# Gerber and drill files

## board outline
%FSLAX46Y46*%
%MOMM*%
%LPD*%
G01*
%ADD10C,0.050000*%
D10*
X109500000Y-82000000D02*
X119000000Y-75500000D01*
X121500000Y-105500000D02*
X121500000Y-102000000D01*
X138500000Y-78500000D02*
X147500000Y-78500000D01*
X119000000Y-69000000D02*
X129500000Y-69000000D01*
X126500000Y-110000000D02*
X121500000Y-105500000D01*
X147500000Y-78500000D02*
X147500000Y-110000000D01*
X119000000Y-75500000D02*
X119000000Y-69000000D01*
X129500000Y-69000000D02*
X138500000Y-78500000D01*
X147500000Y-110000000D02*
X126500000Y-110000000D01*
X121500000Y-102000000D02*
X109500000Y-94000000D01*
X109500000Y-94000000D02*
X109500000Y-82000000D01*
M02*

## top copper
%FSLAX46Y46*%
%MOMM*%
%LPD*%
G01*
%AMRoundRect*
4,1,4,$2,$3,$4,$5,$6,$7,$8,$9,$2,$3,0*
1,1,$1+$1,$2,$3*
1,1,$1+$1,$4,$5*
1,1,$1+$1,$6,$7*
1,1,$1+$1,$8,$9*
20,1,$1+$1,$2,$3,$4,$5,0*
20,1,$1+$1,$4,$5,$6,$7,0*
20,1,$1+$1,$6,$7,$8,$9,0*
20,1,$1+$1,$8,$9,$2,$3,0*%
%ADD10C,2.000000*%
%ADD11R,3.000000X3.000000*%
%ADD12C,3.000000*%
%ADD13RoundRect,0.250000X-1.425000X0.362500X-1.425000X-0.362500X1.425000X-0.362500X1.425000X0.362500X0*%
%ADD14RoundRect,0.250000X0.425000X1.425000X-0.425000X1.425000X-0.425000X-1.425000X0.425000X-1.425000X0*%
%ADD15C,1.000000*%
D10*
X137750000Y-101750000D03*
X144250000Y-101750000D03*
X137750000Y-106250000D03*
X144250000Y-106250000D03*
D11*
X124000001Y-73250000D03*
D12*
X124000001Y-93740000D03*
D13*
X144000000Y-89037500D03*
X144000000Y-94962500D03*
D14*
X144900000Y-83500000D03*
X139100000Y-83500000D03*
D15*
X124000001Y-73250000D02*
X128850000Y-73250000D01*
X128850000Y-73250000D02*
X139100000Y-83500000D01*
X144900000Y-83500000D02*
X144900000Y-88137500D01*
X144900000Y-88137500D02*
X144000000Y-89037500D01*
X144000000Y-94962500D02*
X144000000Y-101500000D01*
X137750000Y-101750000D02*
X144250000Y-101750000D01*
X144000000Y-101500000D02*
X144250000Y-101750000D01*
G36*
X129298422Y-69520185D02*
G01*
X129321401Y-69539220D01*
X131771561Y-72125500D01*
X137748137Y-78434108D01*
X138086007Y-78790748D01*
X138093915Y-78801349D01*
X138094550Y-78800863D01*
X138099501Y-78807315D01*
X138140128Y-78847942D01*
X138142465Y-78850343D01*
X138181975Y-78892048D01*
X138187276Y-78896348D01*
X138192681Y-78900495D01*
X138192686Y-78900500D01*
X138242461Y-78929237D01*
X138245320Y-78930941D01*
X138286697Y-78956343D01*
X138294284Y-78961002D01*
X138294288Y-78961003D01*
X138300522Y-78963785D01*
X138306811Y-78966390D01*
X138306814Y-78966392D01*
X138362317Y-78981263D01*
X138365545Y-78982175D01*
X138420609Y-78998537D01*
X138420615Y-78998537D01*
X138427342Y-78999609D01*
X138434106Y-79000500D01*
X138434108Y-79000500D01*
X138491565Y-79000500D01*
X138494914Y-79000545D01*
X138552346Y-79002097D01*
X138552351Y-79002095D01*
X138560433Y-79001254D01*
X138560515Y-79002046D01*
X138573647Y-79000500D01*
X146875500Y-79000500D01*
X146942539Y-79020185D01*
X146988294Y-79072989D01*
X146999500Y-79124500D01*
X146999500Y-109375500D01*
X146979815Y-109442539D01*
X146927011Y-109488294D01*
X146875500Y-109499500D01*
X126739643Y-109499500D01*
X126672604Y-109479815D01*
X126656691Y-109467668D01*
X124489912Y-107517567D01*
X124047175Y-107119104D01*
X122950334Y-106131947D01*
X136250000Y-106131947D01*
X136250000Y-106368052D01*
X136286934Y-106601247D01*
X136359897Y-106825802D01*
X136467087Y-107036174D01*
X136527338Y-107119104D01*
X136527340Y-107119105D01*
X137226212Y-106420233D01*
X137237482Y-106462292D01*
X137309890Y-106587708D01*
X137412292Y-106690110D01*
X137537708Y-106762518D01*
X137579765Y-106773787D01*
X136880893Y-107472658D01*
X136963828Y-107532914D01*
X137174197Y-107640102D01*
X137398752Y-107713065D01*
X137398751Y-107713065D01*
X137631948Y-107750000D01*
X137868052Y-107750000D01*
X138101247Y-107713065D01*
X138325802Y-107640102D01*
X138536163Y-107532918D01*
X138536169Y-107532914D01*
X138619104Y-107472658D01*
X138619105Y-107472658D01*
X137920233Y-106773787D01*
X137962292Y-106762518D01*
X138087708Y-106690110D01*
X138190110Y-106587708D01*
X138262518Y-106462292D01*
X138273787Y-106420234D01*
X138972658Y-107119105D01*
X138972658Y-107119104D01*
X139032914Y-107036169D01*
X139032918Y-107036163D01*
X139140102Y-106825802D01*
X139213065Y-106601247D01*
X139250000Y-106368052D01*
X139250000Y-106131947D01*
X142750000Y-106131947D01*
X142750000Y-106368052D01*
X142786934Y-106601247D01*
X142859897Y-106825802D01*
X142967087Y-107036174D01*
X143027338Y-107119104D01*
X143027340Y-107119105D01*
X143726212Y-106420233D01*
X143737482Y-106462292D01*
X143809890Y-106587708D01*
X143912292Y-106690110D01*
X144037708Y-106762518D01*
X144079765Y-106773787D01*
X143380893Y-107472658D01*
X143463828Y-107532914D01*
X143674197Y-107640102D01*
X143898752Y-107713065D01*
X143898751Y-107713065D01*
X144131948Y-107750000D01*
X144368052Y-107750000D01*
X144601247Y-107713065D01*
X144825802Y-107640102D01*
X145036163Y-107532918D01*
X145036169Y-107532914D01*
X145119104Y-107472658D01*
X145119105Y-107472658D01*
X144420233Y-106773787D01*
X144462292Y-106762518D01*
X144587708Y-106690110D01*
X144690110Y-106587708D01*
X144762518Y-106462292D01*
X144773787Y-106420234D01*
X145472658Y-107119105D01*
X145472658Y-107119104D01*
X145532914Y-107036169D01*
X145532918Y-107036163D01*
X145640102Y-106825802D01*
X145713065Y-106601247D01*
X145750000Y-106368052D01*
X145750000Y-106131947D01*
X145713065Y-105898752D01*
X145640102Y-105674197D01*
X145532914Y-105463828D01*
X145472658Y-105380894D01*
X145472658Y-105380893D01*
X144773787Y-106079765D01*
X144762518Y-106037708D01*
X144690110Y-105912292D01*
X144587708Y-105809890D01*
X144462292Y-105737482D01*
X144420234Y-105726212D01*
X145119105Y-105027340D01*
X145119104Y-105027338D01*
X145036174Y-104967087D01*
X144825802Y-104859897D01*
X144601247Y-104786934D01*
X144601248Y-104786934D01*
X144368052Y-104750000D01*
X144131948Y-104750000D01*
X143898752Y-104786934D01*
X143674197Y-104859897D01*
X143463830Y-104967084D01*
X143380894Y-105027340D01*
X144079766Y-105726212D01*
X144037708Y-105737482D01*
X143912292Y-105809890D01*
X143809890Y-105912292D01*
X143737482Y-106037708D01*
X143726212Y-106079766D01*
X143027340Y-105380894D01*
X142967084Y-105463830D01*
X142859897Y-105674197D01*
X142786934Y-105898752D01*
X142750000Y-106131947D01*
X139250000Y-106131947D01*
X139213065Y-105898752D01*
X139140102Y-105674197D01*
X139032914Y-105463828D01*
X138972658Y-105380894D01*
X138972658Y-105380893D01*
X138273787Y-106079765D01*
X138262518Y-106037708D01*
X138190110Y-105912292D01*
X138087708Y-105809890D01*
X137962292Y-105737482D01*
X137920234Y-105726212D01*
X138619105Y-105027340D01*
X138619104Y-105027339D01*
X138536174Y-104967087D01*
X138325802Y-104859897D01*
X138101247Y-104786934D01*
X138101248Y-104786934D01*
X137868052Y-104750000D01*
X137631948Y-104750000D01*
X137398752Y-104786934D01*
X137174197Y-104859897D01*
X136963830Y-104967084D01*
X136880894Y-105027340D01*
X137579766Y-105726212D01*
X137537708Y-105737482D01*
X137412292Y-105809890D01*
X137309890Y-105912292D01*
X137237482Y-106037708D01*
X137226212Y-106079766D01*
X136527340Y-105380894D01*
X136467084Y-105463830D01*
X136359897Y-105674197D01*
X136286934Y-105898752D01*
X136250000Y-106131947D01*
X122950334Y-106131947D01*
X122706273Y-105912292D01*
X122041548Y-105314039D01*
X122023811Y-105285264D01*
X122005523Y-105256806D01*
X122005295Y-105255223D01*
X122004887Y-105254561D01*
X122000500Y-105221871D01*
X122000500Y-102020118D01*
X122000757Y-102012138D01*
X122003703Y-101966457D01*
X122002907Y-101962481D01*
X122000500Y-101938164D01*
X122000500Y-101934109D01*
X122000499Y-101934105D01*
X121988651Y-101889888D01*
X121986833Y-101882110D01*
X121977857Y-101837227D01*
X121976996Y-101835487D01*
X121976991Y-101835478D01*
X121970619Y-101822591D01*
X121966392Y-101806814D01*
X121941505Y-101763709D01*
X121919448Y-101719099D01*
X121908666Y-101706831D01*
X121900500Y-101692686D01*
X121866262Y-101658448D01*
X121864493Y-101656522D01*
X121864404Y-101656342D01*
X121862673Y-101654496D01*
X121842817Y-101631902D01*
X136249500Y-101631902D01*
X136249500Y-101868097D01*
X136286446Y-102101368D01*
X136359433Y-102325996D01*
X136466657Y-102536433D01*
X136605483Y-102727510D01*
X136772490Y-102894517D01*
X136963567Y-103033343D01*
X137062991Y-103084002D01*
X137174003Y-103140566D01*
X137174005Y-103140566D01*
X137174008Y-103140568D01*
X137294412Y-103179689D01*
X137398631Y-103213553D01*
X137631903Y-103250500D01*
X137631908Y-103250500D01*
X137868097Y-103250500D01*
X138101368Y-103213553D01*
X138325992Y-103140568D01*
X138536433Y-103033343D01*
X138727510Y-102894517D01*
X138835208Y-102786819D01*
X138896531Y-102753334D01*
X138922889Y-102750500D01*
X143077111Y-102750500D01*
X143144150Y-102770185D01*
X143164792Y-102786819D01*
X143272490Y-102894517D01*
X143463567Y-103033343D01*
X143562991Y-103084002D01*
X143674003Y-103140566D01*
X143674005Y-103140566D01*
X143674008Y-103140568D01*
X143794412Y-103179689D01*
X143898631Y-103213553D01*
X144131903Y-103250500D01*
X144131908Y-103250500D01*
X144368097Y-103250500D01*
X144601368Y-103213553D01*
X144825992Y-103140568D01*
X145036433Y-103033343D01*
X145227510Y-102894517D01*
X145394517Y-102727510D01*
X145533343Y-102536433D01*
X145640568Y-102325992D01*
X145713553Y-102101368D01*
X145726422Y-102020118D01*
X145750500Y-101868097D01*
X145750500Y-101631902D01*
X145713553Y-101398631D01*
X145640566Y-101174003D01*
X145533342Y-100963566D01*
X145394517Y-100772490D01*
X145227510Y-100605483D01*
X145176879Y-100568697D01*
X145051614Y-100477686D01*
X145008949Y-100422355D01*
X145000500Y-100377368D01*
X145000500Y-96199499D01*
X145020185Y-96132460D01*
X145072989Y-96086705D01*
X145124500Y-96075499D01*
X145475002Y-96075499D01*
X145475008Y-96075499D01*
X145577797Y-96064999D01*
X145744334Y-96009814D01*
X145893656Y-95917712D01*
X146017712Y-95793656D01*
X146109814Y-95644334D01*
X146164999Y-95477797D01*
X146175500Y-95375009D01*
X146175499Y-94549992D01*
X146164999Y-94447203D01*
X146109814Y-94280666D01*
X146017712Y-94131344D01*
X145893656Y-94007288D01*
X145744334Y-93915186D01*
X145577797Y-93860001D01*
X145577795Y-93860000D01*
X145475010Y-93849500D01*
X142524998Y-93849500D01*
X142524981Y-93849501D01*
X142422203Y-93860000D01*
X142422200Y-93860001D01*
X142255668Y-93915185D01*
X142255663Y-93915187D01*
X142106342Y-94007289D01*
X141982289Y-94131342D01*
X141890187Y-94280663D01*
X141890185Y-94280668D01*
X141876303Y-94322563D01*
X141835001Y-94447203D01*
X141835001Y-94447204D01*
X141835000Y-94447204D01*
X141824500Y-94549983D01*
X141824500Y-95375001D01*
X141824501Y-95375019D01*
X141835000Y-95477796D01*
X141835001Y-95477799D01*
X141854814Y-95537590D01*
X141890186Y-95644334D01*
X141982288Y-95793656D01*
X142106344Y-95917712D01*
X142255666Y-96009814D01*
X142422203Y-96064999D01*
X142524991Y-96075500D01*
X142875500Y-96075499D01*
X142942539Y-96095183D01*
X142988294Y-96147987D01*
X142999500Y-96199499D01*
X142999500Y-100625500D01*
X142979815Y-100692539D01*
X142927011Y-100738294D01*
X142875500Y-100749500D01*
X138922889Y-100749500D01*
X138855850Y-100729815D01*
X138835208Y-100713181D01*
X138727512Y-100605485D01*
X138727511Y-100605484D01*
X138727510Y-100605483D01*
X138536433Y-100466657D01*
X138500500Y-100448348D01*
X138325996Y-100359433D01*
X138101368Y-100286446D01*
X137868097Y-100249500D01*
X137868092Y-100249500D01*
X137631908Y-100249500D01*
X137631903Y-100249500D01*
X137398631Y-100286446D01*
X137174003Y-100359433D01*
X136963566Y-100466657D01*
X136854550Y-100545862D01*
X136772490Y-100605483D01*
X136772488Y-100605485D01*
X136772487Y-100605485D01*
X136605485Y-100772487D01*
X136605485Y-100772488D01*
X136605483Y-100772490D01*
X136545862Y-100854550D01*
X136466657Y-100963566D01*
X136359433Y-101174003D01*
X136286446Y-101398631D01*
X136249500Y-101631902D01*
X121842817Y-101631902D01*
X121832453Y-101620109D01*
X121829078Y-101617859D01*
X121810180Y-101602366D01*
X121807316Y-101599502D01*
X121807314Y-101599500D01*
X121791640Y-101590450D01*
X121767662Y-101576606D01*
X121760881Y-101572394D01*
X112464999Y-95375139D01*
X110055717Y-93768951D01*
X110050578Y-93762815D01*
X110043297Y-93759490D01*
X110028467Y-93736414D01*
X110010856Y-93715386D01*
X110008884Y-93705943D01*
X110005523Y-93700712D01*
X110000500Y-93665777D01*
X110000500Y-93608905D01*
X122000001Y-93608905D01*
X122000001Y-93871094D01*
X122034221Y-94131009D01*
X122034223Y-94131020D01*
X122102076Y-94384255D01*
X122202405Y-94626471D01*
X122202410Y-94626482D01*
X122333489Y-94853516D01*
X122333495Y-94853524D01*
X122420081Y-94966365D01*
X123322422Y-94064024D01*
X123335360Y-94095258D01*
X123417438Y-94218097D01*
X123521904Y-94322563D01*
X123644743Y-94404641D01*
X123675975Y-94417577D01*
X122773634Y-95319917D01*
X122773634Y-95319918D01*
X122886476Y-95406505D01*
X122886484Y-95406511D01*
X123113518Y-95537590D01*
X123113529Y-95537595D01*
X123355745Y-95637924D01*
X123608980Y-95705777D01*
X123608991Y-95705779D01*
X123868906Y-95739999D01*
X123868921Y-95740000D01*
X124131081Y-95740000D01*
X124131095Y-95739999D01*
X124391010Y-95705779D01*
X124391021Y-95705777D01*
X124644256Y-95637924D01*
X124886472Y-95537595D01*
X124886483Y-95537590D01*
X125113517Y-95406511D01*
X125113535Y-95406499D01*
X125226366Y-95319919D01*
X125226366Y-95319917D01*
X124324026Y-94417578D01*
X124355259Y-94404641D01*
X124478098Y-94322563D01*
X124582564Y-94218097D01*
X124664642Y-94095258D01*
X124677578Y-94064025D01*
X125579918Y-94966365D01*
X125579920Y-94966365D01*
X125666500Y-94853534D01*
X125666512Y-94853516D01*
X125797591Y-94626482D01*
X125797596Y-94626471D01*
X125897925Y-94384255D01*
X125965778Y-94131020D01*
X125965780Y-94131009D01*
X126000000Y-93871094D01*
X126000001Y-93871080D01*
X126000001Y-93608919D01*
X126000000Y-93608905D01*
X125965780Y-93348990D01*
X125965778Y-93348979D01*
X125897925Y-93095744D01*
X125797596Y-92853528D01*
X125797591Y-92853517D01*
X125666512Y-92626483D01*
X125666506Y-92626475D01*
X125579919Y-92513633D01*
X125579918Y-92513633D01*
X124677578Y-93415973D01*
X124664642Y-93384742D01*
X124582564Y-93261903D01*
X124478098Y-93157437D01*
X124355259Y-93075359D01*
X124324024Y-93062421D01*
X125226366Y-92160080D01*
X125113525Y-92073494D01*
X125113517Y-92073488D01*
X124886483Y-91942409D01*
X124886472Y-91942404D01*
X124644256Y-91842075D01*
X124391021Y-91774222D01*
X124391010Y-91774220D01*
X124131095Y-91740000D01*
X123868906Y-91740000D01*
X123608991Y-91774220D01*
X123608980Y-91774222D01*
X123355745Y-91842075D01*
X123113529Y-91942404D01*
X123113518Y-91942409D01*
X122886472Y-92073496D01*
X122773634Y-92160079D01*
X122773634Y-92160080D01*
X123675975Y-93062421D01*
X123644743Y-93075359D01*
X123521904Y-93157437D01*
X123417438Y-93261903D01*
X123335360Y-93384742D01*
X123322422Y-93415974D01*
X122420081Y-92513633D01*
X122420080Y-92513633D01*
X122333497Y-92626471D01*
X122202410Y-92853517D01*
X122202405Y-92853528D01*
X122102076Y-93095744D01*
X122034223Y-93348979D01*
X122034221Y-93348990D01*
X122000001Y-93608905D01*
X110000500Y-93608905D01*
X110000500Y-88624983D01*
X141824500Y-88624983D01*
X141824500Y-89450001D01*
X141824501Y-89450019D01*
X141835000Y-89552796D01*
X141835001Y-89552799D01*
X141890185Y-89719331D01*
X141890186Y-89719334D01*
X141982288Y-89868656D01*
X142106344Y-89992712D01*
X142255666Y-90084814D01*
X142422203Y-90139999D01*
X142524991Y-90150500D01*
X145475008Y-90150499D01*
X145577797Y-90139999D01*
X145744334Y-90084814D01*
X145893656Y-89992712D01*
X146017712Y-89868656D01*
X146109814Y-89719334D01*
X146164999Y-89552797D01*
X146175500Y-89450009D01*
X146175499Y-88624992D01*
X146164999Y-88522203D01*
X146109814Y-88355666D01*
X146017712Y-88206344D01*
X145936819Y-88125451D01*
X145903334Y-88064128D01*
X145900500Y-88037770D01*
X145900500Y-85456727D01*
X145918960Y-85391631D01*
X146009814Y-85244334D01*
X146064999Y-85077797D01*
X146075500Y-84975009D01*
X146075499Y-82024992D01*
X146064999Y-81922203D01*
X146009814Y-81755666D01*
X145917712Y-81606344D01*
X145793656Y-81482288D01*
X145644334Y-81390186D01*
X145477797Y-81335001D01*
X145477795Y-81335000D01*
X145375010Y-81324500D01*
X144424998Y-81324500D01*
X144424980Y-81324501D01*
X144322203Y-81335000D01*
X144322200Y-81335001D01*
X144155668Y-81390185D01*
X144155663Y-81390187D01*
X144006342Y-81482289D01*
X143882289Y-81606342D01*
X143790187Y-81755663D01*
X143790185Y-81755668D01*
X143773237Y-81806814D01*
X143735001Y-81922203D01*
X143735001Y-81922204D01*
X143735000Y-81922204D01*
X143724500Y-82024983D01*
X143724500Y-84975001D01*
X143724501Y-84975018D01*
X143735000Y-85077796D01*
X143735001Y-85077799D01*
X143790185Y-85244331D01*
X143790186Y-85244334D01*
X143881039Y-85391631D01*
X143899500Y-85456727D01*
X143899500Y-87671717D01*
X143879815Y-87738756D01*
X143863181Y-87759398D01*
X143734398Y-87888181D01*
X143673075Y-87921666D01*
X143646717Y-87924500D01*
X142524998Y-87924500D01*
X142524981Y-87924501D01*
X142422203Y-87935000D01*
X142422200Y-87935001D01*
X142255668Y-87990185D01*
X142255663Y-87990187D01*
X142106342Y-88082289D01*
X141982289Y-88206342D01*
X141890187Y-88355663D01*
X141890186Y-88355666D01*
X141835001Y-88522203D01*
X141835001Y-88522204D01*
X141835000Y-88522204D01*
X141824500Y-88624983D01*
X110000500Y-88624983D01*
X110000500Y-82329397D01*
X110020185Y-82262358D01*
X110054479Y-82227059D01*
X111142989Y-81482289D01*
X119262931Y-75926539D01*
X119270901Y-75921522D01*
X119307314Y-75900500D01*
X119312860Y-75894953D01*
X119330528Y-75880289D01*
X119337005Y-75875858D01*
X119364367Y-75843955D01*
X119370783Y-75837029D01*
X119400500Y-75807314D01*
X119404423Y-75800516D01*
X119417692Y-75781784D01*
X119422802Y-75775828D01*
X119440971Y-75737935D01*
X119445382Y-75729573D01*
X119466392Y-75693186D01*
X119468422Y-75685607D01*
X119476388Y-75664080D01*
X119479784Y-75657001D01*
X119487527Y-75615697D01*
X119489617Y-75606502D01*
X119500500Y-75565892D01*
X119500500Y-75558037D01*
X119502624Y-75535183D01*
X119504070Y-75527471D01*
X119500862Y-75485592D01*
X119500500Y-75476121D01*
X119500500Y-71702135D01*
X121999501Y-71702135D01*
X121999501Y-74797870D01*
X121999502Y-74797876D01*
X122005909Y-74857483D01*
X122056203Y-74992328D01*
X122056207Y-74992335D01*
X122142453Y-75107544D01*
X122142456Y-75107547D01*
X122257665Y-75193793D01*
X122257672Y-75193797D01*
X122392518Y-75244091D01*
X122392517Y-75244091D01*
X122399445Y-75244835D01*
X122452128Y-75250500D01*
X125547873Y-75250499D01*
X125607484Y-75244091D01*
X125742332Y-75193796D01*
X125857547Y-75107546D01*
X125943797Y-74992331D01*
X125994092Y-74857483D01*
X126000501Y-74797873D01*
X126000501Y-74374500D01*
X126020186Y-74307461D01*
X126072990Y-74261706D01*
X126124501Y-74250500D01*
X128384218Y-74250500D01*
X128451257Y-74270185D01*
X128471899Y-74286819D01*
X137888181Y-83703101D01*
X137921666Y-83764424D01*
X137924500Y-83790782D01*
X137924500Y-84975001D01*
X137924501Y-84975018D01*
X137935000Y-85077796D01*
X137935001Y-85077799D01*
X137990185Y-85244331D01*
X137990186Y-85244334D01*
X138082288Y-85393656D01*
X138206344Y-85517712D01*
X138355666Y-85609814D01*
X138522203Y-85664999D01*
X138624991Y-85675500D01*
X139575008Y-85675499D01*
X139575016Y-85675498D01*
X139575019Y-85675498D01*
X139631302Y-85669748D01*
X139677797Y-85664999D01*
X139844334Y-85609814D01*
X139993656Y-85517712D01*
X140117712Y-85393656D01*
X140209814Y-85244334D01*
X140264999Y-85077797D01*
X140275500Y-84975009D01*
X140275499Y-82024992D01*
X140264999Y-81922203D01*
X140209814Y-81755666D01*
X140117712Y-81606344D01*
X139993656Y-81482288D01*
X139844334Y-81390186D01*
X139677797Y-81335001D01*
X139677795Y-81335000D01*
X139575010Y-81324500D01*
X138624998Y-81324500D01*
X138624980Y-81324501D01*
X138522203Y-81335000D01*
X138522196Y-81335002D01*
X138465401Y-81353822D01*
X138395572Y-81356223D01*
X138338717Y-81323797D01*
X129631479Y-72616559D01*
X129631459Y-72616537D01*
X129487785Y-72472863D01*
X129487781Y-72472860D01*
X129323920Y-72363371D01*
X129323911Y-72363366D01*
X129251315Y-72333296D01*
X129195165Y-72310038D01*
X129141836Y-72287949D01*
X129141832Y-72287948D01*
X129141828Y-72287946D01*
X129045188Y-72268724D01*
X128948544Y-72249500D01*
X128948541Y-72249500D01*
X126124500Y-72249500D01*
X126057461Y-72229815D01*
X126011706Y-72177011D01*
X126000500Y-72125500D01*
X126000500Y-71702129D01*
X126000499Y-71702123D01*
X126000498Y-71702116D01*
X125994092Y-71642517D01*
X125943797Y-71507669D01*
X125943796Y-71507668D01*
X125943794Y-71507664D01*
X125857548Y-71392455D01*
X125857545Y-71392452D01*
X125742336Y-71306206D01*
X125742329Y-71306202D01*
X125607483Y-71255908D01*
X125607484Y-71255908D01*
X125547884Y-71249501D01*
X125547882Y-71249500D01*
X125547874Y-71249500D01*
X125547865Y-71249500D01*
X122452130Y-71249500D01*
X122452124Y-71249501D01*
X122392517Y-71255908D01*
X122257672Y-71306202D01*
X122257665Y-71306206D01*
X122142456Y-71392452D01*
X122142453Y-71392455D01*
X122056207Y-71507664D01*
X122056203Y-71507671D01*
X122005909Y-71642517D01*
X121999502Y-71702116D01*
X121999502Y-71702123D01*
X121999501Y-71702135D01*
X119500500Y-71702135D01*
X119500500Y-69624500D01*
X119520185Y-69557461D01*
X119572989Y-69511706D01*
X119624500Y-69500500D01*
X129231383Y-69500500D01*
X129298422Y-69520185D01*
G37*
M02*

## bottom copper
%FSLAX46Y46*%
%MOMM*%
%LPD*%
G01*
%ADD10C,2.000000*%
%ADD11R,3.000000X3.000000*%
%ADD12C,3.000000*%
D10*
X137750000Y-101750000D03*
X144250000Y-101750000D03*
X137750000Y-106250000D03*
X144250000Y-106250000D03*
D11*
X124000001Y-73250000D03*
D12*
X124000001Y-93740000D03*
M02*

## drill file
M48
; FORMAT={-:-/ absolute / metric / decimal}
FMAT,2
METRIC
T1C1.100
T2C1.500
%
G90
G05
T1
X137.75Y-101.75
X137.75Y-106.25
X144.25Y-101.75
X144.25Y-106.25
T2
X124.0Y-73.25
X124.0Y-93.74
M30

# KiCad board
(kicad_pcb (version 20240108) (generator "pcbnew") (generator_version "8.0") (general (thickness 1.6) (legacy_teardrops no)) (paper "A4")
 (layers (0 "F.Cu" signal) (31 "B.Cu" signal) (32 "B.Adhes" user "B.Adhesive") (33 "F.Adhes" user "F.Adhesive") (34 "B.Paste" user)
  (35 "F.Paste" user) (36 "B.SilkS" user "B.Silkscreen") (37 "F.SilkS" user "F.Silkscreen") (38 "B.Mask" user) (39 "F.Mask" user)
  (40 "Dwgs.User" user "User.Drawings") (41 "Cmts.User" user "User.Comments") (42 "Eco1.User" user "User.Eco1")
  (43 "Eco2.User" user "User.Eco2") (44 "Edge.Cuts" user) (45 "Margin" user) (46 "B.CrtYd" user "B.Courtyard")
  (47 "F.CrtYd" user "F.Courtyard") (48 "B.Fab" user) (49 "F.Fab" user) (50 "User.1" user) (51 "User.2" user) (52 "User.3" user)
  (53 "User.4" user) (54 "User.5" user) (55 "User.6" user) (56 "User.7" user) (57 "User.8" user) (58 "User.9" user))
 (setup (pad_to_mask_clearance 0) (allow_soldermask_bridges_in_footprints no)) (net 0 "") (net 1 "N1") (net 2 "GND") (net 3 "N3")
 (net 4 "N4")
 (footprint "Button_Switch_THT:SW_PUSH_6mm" (layer "F.Cu") (at 137.75 101.75)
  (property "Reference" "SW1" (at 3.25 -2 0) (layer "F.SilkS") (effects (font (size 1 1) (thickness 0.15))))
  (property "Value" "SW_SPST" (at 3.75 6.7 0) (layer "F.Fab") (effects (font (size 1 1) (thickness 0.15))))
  (pad "1" thru_hole circle (at 0 0 90) (size 2 2) (drill 1.1) (layers "*.Cu" "*.Mask") (remove_unused_layers no) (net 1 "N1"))
  (pad "1" thru_hole circle (at 6.5 0 90) (size 2 2) (drill 1.1) (layers "*.Cu" "*.Mask") (remove_unused_layers no) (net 1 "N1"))
  (pad "2" thru_hole circle (at 0 4.5 90) (size 2 2) (drill 1.1) (layers "*.Cu" "*.Mask") (remove_unused_layers no) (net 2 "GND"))
  (pad "2" thru_hole circle (at 6.5 4.5 90) (size 2 2) (drill 1.1) (layers "*.Cu" "*.Mask") (remove_unused_layers no) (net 2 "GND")))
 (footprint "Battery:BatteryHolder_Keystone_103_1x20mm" (layer "F.Cu") (at 124.000001 73.25 -90)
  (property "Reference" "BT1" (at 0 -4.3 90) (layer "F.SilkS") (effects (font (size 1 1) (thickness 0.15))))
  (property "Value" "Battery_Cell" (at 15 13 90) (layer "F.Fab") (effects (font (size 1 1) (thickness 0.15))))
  (pad "1" thru_hole rect (at 0 0 270) (size 3 3) (drill 1.5) (layers "*.Cu" "*.Mask") (remove_unused_layers no) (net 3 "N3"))
  (pad "2" thru_hole circle (at 20.49 0 270) (size 3 3) (drill 1.5) (layers "*.Cu" "*.Mask") (remove_unused_layers no) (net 2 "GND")))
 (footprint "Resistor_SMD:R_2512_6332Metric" (layer "F.Cu") (at 144 92 -90)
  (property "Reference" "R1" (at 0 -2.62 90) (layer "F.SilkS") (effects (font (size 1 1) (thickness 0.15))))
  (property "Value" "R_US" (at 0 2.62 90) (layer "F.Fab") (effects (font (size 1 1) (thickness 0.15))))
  (pad "1" smd roundrect (at -2.9625 0 270) (size 1.225 3.35) (layers "F.Cu" "F.Paste" "F.Mask") (roundrect_rratio 0.204082) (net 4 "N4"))
  (pad "2" smd roundrect (at 2.9625 0 270) (size 1.225 3.35) (layers "F.Cu" "F.Paste" "F.Mask") (roundrect_rratio 0.204082) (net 1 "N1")))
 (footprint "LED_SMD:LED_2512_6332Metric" (layer "F.Cu") (at 142 83.5 180)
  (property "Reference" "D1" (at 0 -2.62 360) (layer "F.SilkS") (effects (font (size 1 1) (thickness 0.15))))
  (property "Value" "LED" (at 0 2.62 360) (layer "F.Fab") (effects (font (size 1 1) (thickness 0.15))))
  (pad "1" smd roundrect (at -2.9 0 180) (size 1.35 3.35) (layers "F.Cu" "F.Paste" "F.Mask") (roundrect_rratio 0.185185) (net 4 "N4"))
  (pad "2" smd roundrect (at 2.9 0 180) (size 1.35 3.35) (layers "F.Cu" "F.Paste" "F.Mask") (roundrect_rratio 0.185185) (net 3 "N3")))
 (gr_line (start 109.5 82) (end 119 75.5) (stroke (width 0.05) (type default)) (layer "Edge.Cuts"))
 (gr_line (start 121.5 105.5) (end 121.5 102) (stroke (width 0.05) (type default)) (layer "Edge.Cuts"))
 (gr_line (start 138.5 78.5) (end 147.5 78.5) (stroke (width 0.05) (type default)) (layer "Edge.Cuts"))
 (gr_line (start 119 69) (end 129.5 69) (stroke (width 0.05) (type default)) (layer "Edge.Cuts"))
 (gr_line (start 126.5 110) (end 121.5 105.5) (stroke (width 0.05) (type default)) (layer "Edge.Cuts"))
 (gr_line (start 147.5 78.5) (end 147.5 110) (stroke (width 0.05) (type default)) (layer "Edge.Cuts"))
 (gr_line (start 119 75.5) (end 119 69) (stroke (width 0.05) (type default)) (layer "Edge.Cuts"))
 (gr_line (start 129.5 69) (end 138.5 78.5) (stroke (width 0.05) (type default)) (layer "Edge.Cuts"))
 (gr_line (start 147.5 110) (end 126.5 110) (stroke (width 0.05) (type default)) (layer "Edge.Cuts"))
 (gr_line (start 121.5 102) (end 109.5 94) (stroke (width 0.05) (type default)) (layer "Edge.Cuts"))
 (gr_line (start 109.5 94) (end 109.5 82) (stroke (width 0.05) (type default)) (layer "Edge.Cuts"))
 (segment (start 124.000001 73.25) (end 128.85 73.25) (width 1) (layer "F.Cu") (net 3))
 (segment (start 128.85 73.25) (end 139.1 83.5) (width 1) (layer "F.Cu") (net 3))
 (segment (start 144.9 83.5) (end 144.9 88.1375) (width 1) (layer "F.Cu") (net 4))
 (segment (start 144.9 88.1375) (end 144 89.0375) (width 1) (layer "F.Cu") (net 4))
 (segment (start 144 94.9625) (end 144 101.5) (width 1) (layer "F.Cu") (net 1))
 (segment (start 137.75 101.75) (end 144.25 101.75) (width 1) (layer "F.Cu") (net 1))
 (segment (start 144 101.5) (end 144.25 101.75) (width 1) (layer "F.Cu") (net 1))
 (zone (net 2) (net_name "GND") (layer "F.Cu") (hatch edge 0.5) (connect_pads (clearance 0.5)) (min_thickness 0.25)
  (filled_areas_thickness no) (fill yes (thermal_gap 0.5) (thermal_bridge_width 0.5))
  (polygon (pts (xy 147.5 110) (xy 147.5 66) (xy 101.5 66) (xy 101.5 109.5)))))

